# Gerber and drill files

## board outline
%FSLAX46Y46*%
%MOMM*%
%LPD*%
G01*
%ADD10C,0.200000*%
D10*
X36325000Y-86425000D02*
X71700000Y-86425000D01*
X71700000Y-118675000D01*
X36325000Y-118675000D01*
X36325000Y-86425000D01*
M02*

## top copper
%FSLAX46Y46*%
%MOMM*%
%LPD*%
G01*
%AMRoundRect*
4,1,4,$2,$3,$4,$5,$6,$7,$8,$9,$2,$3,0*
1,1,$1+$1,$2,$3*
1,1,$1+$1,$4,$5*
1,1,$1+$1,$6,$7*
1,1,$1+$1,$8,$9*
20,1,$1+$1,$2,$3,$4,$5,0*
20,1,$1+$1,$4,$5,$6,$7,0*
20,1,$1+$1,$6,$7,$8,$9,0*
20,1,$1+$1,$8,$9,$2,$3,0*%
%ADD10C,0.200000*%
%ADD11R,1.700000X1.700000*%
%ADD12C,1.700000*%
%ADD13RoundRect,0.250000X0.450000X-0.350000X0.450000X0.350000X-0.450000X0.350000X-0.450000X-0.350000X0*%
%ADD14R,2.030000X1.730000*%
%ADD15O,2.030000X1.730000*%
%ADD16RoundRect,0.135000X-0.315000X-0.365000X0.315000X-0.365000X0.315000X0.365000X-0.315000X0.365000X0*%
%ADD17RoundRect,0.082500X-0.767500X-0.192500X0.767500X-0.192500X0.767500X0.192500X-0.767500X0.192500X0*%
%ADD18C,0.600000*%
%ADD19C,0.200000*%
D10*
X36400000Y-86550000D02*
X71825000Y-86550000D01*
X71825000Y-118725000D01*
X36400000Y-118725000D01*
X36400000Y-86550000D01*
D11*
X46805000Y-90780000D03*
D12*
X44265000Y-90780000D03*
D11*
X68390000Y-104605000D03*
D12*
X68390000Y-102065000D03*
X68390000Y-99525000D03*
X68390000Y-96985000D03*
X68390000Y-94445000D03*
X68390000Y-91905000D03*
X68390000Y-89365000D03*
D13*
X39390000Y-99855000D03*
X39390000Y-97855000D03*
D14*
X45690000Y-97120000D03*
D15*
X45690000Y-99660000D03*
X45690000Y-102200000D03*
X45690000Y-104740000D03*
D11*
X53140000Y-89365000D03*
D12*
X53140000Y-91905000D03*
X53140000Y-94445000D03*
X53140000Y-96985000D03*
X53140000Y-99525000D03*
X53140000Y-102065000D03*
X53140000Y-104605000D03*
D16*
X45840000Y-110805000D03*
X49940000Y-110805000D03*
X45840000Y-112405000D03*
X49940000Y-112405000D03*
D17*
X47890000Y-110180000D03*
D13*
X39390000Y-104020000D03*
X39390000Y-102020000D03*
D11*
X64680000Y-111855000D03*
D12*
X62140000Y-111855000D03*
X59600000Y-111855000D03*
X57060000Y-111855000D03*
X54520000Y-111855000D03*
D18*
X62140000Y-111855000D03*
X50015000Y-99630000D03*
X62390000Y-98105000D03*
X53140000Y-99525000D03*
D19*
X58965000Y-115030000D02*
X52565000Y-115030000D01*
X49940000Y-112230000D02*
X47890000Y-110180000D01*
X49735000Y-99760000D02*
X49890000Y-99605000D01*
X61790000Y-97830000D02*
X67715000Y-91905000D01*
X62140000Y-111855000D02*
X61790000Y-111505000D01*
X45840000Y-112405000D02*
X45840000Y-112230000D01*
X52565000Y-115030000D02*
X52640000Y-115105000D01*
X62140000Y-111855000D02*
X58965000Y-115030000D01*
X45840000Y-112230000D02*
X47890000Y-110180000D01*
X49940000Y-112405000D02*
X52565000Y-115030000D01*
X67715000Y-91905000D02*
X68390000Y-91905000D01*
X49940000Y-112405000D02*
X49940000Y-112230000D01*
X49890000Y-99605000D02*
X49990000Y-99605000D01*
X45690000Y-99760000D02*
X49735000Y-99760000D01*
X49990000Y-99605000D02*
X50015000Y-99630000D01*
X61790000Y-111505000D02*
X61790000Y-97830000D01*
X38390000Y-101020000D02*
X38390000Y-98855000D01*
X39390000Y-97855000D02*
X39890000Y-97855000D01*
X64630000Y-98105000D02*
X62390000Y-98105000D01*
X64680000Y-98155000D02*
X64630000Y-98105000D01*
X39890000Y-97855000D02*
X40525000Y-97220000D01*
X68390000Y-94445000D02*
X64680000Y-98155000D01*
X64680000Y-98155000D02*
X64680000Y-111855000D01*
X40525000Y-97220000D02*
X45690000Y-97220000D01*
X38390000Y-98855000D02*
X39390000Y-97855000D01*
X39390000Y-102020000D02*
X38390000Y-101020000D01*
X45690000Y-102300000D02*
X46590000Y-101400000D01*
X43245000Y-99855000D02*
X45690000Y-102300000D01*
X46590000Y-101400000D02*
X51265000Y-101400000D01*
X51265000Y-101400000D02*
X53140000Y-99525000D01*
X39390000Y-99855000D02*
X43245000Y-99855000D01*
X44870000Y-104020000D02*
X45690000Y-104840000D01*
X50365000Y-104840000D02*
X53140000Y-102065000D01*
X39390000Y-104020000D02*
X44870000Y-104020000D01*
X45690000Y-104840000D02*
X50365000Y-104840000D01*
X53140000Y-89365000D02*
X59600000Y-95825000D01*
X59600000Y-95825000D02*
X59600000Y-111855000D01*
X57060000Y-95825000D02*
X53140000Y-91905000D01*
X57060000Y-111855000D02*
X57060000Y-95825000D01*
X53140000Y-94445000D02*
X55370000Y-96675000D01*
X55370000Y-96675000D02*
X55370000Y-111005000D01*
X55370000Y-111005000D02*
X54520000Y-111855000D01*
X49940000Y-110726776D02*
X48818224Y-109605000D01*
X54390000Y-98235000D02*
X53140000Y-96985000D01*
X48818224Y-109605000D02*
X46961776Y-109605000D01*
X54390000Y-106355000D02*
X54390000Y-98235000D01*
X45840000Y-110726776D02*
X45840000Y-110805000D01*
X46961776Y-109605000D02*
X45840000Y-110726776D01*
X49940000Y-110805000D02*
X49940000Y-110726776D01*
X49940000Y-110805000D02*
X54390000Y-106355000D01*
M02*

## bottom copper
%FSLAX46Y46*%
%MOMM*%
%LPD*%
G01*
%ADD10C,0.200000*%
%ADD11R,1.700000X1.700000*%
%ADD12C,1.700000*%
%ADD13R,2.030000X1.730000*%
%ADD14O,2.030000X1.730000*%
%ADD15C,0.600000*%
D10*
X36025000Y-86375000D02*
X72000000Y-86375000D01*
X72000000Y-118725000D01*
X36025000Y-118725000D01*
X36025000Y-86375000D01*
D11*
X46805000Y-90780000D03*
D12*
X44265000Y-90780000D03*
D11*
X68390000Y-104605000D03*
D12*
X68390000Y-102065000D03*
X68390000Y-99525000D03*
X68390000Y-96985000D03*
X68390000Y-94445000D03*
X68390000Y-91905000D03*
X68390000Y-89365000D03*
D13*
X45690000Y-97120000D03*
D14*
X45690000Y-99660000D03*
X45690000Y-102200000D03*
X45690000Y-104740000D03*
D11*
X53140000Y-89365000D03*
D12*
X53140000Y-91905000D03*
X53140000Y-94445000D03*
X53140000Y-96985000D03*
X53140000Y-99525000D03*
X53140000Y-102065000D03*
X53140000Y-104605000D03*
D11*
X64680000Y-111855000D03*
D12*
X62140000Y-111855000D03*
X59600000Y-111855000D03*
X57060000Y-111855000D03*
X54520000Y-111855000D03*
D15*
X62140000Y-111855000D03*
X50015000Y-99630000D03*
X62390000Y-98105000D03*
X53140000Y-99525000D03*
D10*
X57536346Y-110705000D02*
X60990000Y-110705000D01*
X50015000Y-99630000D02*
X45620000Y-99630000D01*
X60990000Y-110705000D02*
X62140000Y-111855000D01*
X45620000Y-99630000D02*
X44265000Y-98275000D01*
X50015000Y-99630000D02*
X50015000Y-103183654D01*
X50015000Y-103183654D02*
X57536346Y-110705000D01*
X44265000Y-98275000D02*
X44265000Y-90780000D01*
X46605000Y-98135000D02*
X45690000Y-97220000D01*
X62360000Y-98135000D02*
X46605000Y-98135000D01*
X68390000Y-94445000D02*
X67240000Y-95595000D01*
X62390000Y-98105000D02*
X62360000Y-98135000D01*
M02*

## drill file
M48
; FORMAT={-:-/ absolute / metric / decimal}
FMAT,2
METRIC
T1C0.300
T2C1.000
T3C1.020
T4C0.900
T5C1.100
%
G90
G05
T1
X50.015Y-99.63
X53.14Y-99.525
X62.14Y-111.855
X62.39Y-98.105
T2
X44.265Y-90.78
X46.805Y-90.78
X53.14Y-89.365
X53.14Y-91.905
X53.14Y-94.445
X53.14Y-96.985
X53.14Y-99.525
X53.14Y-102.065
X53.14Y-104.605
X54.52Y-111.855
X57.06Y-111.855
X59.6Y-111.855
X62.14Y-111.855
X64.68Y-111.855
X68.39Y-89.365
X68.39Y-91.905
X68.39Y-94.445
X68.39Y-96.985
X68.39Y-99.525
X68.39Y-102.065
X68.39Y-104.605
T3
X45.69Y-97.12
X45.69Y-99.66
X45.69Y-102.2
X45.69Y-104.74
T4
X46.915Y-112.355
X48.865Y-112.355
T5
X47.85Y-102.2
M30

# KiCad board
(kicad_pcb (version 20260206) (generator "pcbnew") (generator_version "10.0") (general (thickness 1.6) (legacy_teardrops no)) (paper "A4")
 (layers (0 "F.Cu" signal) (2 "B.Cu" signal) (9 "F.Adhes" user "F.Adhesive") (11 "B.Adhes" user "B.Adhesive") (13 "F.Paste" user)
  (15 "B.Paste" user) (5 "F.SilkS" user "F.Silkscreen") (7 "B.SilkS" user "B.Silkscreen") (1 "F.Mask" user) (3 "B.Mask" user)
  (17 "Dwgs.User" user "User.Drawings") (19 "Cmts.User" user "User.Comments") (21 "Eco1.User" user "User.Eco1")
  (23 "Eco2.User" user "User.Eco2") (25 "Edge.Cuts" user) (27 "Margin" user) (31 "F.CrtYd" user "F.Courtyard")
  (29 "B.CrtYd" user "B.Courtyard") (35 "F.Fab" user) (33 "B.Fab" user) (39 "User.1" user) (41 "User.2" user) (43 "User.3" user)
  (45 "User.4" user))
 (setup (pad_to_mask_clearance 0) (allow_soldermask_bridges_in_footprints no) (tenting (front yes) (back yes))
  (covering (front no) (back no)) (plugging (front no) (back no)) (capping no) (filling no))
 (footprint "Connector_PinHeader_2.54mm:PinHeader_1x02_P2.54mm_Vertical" (layer "F.Cu") (at 46.805 90.78 -90)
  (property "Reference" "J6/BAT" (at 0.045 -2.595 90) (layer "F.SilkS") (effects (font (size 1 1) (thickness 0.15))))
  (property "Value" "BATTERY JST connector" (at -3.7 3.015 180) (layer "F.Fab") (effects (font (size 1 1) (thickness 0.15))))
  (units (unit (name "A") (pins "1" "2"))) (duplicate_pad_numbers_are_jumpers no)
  (pad "1" thru_hole rect (at 0 0 270) (size 1.7 1.7) (drill 1) (layers "*.Cu" "*.Mask") (remove_unused_layers no) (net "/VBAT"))
  (pad "2" thru_hole circle (at 0 2.54 270) (size 1.7 1.7) (drill 1) (layers "*.Cu" "*.Mask") (remove_unused_layers no) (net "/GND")))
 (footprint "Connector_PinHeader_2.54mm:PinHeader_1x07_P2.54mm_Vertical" (layer "F.Cu") (at 68.39 104.605 180)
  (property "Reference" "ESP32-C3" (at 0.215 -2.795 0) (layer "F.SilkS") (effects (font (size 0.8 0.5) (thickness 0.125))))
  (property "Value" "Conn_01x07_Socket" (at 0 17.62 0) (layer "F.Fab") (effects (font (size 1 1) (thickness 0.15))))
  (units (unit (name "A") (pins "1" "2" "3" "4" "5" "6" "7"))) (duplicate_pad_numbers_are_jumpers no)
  (pad "1" thru_hole rect (at 0 0 180) (size 1.7 1.7) (drill 1) (layers "*.Cu" "*.Mask") (remove_unused_layers no) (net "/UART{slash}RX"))
  (pad "2" thru_hole circle (at 0 2.54 180) (size 1.7 1.7) (drill 1) (layers "*.Cu" "*.Mask") (remove_unused_layers no)
   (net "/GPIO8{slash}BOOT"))
  (pad "3" thru_hole circle (at 0 5.08 180) (size 1.7 1.7) (drill 1) (layers "*.Cu" "*.Mask") (remove_unused_layers no)
   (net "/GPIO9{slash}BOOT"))
  (pad "4" thru_hole circle (at 0 7.62 180) (size 1.7 1.7) (drill 1) (layers "*.Cu" "*.Mask") (remove_unused_layers no) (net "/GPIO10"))
  (pad "5" thru_hole circle (at 0 10.16 180) (size 1.7 1.7) (drill 1) (layers "*.Cu" "*.Mask") (remove_unused_layers no) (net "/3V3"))
  (pad "6" thru_hole circle (at 0 12.7 180) (size 1.7 1.7) (drill 1) (layers "*.Cu" "*.Mask") (remove_unused_layers no) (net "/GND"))
  (pad "7" thru_hole circle (at 0 15.24 180) (size 1.7 1.7) (drill 1) (layers "*.Cu" "*.Mask") (remove_unused_layers no) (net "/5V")))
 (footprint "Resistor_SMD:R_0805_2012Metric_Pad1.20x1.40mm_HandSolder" (layer "F.Cu") (at 39.39 98.855 90)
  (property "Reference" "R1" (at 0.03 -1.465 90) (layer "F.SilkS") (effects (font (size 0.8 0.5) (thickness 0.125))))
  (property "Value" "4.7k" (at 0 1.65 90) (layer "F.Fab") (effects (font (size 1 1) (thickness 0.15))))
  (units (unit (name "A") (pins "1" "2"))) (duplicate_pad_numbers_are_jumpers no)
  (pad "1" smd roundrect (at -1 0 90) (size 1.2 1.4) (layers "F.Cu" "F.Mask" "F.Paste") (roundrect_rratio 0.208333) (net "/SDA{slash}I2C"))
  (pad "2" smd roundrect (at 1 0 90) (size 1.2 1.4) (layers "F.Cu" "F.Mask" "F.Paste") (roundrect_rratio 0.208333) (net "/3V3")))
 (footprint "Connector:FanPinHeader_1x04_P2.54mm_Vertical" (layer "F.Cu") (at 45.69 97.12 -90)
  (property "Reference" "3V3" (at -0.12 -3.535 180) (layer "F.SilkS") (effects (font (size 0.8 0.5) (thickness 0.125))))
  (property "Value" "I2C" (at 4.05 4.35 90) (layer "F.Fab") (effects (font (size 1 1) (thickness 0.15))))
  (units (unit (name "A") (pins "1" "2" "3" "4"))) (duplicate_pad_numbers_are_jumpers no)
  (pad "" np_thru_hole circle (at 5.08 -2.16) (size 1.1 1.1) (drill 1.1) (layers "*.Cu" "*.Mask"))
  (pad "1" thru_hole rect (at 0 0) (size 2.03 1.73) (drill 1.02) (layers "*.Cu" "*.Mask") (remove_unused_layers no) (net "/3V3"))
  (pad "2" thru_hole oval (at 2.54 0) (size 2.03 1.73) (drill 1.02) (layers "*.Cu" "*.Mask") (remove_unused_layers no) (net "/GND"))
  (pad "3" thru_hole oval (at 5.08 0) (size 2.03 1.73) (drill 1.02) (layers "*.Cu" "*.Mask") (remove_unused_layers no)
   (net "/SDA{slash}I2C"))
  (pad "4" thru_hole oval (at 7.62 0) (size 2.03 1.73) (drill 1.02) (layers "*.Cu" "*.Mask") (remove_unused_layers no)
   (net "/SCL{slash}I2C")))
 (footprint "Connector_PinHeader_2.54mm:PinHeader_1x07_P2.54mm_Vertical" (layer "F.Cu") (at 53.14 89.365)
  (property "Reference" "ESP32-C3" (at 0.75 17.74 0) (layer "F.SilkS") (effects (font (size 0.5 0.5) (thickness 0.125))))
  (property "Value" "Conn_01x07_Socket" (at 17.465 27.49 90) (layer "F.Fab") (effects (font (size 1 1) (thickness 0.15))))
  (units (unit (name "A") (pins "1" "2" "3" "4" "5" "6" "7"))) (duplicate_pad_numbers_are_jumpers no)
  (pad "1" thru_hole rect (at 0 0) (size 1.7 1.7) (drill 1) (layers "*.Cu" "*.Mask") (remove_unused_layers no) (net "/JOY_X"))
  (pad "2" thru_hole circle (at 0 2.54) (size 1.7 1.7) (drill 1) (layers "*.Cu" "*.Mask") (remove_unused_layers no) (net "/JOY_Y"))
  (pad "3" thru_hole circle (at 0 5.08) (size 1.7 1.7) (drill 1) (layers "*.Cu" "*.Mask") (remove_unused_layers no) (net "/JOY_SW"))
  (pad "4" thru_hole circle (at 0 7.62) (size 1.7 1.7) (drill 1) (layers "*.Cu" "*.Mask") (remove_unused_layers no) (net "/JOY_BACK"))
  (pad "5" thru_hole circle (at 0 10.16) (size 1.7 1.7) (drill 1) (layers "*.Cu" "*.Mask") (remove_unused_layers no) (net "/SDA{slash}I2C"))
  (pad "6" thru_hole circle (at 0 12.7) (size 1.7 1.7) (drill 1) (layers "*.Cu" "*.Mask") (remove_unused_layers no) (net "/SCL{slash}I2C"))
  (pad "7" thru_hole circle (at 0 15.24) (size 1.7 1.7) (drill 1) (layers "*.Cu" "*.Mask") (remove_unused_layers no) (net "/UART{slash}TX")))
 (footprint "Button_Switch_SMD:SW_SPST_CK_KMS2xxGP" (layer "F.Cu") (at 47.89 111.605)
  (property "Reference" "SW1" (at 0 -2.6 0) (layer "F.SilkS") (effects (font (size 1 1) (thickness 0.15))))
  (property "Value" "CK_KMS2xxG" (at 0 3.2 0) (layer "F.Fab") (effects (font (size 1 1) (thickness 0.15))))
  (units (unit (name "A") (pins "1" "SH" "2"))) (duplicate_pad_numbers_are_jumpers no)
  (pad "" np_thru_hole circle (at -0.975 0.75) (size 0.9 0.9) (drill 0.9) (layers "*.Cu" "*.Mask"))
  (pad "" np_thru_hole circle (at 0.975 0.75) (size 0.9 0.9) (drill 0.9) (layers "*.Cu" "*.Mask"))
  (pad "1" smd roundrect (at -2.05 -0.8) (size 0.9 1) (layers "F.Cu" "F.Mask" "F.Paste") (roundrect_rratio 0.15) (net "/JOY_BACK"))
  (pad "1" smd roundrect (at 2.05 -0.8) (size 0.9 1) (layers "F.Cu" "F.Mask" "F.Paste") (roundrect_rratio 0.15) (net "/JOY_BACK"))
  (pad "2" smd roundrect (at -2.05 0.8) (size 0.9 1) (layers "F.Cu" "F.Mask" "F.Paste") (roundrect_rratio 0.15) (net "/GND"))
  (pad "2" smd roundrect (at 2.05 0.8) (size 0.9 1) (layers "F.Cu" "F.Mask" "F.Paste") (roundrect_rratio 0.15) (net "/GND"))
  (pad "SH" smd roundrect (at 0 -1.425) (size 1.7 0.55) (layers "F.Cu" "F.Mask" "F.Paste") (roundrect_rratio 0.15) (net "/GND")))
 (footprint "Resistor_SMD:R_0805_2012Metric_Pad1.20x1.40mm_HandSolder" (layer "F.Cu") (at 39.39 103.02 90)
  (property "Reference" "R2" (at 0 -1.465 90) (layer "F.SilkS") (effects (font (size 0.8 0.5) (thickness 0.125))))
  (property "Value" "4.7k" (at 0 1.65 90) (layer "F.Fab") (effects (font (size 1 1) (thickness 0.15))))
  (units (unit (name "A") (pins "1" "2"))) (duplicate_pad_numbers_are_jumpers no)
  (pad "1" smd roundrect (at -1 0 90) (size 1.2 1.4) (layers "F.Cu" "F.Mask" "F.Paste") (roundrect_rratio 0.208333) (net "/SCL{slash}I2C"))
  (pad "2" smd roundrect (at 1 0 90) (size 1.2 1.4) (layers "F.Cu" "F.Mask" "F.Paste") (roundrect_rratio 0.208333) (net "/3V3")))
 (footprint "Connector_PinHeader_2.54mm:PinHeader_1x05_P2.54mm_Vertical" (layer "F.Cu") (at 64.68 111.855 -90)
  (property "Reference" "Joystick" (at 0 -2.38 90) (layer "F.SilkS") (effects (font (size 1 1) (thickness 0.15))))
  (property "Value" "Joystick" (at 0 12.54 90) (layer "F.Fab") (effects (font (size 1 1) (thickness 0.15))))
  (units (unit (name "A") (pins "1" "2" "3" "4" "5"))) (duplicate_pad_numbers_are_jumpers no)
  (pad "1" thru_hole rect (at 0 0 270) (size 1.7 1.7) (drill 1) (layers "*.Cu" "*.Mask") (remove_unused_layers no) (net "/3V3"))
  (pad "2" thru_hole circle (at 0 2.54 270) (size 1.7 1.7) (drill 1) (layers "*.Cu" "*.Mask") (remove_unused_layers no) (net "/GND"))
  (pad "3" thru_hole circle (at 0 5.08 270) (size 1.7 1.7) (drill 1) (layers "*.Cu" "*.Mask") (remove_unused_layers no) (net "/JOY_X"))
  (pad "4" thru_hole circle (at 0 7.62 270) (size 1.7 1.7) (drill 1) (layers "*.Cu" "*.Mask") (remove_unused_layers no) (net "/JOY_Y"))
  (pad "5" thru_hole circle (at 0 10.16 270) (size 1.7 1.7) (drill 1) (layers "*.Cu" "*.Mask") (remove_unused_layers no) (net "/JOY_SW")))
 (gr_rect (start 36.4 86.55) (end 71.825 118.725) (stroke (width 0.2) (type default)) (fill no) (layer "F.Cu"))
 (gr_rect (start 36.025 86.375) (end 72 118.725) (stroke (width 0.2) (type solid)) (fill no) (layer "B.Cu") (net "/GND"))
 (gr_rect (start 36.325 86.425) (end 71.7 118.675) (stroke (width 0.2) (type solid)) (fill no) (layer "Edge.Cuts"))
 (segment (start 58.965 115.03) (end 52.565 115.03) (width 0.2) (layer "F.Cu") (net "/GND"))
 (segment (start 49.94 112.23) (end 47.89 110.18) (width 0.2) (layer "F.Cu") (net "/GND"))
 (segment (start 49.735 99.76) (end 49.89 99.605) (width 0.2) (layer "F.Cu") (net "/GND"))
 (segment (start 61.79 97.83) (end 67.715 91.905) (width 0.2) (layer "F.Cu") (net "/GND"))
 (segment (start 62.14 111.855) (end 61.79 111.505) (width 0.2) (layer "F.Cu") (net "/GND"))
 (segment (start 45.84 112.405) (end 45.84 112.23) (width 0.2) (layer "F.Cu") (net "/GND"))
 (segment (start 52.565 115.03) (end 52.64 115.105) (width 0.2) (layer "F.Cu") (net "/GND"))
 (segment (start 62.14 111.855) (end 58.965 115.03) (width 0.2) (layer "F.Cu") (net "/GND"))
 (segment (start 45.84 112.23) (end 47.89 110.18) (width 0.2) (layer "F.Cu") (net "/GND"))
 (segment (start 49.94 112.405) (end 52.565 115.03) (width 0.2) (layer "F.Cu") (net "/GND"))
 (segment (start 67.715 91.905) (end 68.39 91.905) (width 0.2) (layer "F.Cu") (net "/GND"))
 (segment (start 49.94 112.405) (end 49.94 112.23) (width 0.2) (layer "F.Cu") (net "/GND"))
 (segment (start 49.89 99.605) (end 49.99 99.605) (width 0.2) (layer "F.Cu") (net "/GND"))
 (segment (start 45.69 99.76) (end 49.735 99.76) (width 0.2) (layer "F.Cu") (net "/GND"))
 (segment (start 49.99 99.605) (end 50.015 99.63) (width 0.2) (layer "F.Cu") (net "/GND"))
 (segment (start 61.79 111.505) (end 61.79 97.83) (width 0.2) (layer "F.Cu") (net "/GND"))
 (via (at 62.14 111.855) (size 0.6) (drill 0.3) (layers "F.Cu" "B.Cu") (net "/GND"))
 (via (at 50.015 99.63) (size 0.6) (drill 0.3) (layers "F.Cu" "B.Cu") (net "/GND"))
 (segment (start 57.536346 110.705) (end 60.99 110.705) (width 0.2) (layer "B.Cu") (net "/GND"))
 (segment (start 50.015 99.63) (end 45.62 99.63) (width 0.2) (layer "B.Cu") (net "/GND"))
 (segment (start 60.99 110.705) (end 62.14 111.855) (width 0.2) (layer "B.Cu") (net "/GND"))
 (segment (start 45.62 99.63) (end 44.265 98.275) (width 0.2) (layer "B.Cu") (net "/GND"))
 (segment (start 50.015 99.63) (end 50.015 103.183654) (width 0.2) (layer "B.Cu") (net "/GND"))
 (segment (start 50.015 103.183654) (end 57.536346 110.705) (width 0.2) (layer "B.Cu") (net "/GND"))
 (segment (start 44.265 98.275) (end 44.265 90.78) (width 0.2) (layer "B.Cu") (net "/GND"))
 (segment (start 38.39 101.02) (end 38.39 98.855) (width 0.2) (layer "F.Cu") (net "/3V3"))
 (segment (start 39.39 97.855) (end 39.89 97.855) (width 0.2) (layer "F.Cu") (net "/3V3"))
 (segment (start 64.63 98.105) (end 62.39 98.105) (width 0.2) (layer "F.Cu") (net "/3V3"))
 (segment (start 64.68 98.155) (end 64.63 98.105) (width 0.2) (layer "F.Cu") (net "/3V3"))
 (segment (start 39.89 97.855) (end 40.525 97.22) (width 0.2) (layer "F.Cu") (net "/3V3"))
 (segment (start 68.39 94.445) (end 64.68 98.155) (width 0.2) (layer "F.Cu") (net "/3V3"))
 (segment (start 64.68 98.155) (end 64.68 111.855) (width 0.2) (layer "F.Cu") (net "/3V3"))
 (segment (start 40.525 97.22) (end 45.69 97.22) (width 0.2) (layer "F.Cu") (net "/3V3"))
 (segment (start 38.39 98.855) (end 39.39 97.855) (width 0.2) (layer "F.Cu") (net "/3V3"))
 (segment (start 39.39 102.02) (end 38.39 101.02) (width 0.2) (layer "F.Cu") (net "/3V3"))
 (via (at 62.39 98.105) (size 0.6) (drill 0.3) (layers "F.Cu" "B.Cu") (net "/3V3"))
 (segment (start 46.605 98.135) (end 45.69 97.22) (width 0.2) (layer "B.Cu") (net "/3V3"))
 (segment (start 62.36 98.135) (end 46.605 98.135) (width 0.2) (layer "B.Cu") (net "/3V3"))
 (segment (start 68.39 94.445) (end 67.24 95.595) (width 0.2) (layer "B.Cu") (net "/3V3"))
 (segment (start 62.39 98.105) (end 62.36 98.135) (width 0.2) (layer "B.Cu") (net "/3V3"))
 (segment (start 45.69 102.3) (end 46.59 101.4) (width 0.2) (layer "F.Cu") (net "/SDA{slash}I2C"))
 (segment (start 43.245 99.855) (end 45.69 102.3) (width 0.2) (layer "F.Cu") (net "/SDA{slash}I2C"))
 (segment (start 46.59 101.4) (end 51.265 101.4) (width 0.2) (layer "F.Cu") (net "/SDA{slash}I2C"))
 (segment (start 51.265 101.4) (end 53.14 99.525) (width 0.2) (layer "F.Cu") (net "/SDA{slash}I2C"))
 (segment (start 39.39 99.855) (end 43.245 99.855) (width 0.2) (layer "F.Cu") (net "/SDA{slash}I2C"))
 (via (at 53.14 99.525) (size 0.6) (drill 0.3) (layers "F.Cu" "B.Cu") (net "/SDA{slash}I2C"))
 (segment (start 44.87 104.02) (end 45.69 104.84) (width 0.2) (layer "F.Cu") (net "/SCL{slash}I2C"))
 (segment (start 50.365 104.84) (end 53.14 102.065) (width 0.2) (layer "F.Cu") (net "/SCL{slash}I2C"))
 (segment (start 39.39 104.02) (end 44.87 104.02) (width 0.2) (layer "F.Cu") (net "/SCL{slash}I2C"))
 (segment (start 45.69 104.84) (end 50.365 104.84) (width 0.2) (layer "F.Cu") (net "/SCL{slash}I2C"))
 (segment (start 53.14 89.365) (end 59.6 95.825) (width 0.2) (layer "F.Cu") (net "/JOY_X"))
 (segment (start 59.6 95.825) (end 59.6 111.855) (width 0.2) (layer "F.Cu") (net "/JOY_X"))
 (segment (start 57.06 95.825) (end 53.14 91.905) (width 0.2) (layer "F.Cu") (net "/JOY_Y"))
 (segment (start 57.06 111.855) (end 57.06 95.825) (width 0.2) (layer "F.Cu") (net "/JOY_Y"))
 (segment (start 53.14 94.445) (end 55.37 96.675) (width 0.2) (layer "F.Cu") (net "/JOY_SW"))
 (segment (start 55.37 96.675) (end 55.37 111.005) (width 0.2) (layer "F.Cu") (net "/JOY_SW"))
 (segment (start 55.37 111.005) (end 54.52 111.855) (width 0.2) (layer "F.Cu") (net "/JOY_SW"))
 (segment (start 49.94 110.726776) (end 48.818224 109.605) (width 0.2) (layer "F.Cu") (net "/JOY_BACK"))
 (segment (start 54.39 98.235) (end 53.14 96.985) (width 0.2) (layer "F.Cu") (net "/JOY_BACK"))
 (segment (start 48.818224 109.605) (end 46.961776 109.605) (width 0.2) (layer "F.Cu") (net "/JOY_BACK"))
 (segment (start 54.39 106.355) (end 54.39 98.235) (width 0.2) (layer "F.Cu") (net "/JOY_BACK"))
 (segment (start 45.84 110.726776) (end 45.84 110.805) (width 0.2) (layer "F.Cu") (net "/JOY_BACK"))
 (segment (start 46.961776 109.605) (end 45.84 110.726776) (width 0.2) (layer "F.Cu") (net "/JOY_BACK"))
 (segment (start 49.94 110.805) (end 49.94 110.726776) (width 0.2) (layer "F.Cu") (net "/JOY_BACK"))
 (segment (start 49.94 110.805) (end 54.39 106.355) (width 0.2) (layer "F.Cu") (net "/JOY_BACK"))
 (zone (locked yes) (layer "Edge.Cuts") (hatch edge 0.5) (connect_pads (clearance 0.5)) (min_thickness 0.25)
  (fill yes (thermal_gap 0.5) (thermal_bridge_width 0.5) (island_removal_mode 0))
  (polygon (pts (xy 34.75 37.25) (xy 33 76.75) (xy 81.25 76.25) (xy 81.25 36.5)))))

